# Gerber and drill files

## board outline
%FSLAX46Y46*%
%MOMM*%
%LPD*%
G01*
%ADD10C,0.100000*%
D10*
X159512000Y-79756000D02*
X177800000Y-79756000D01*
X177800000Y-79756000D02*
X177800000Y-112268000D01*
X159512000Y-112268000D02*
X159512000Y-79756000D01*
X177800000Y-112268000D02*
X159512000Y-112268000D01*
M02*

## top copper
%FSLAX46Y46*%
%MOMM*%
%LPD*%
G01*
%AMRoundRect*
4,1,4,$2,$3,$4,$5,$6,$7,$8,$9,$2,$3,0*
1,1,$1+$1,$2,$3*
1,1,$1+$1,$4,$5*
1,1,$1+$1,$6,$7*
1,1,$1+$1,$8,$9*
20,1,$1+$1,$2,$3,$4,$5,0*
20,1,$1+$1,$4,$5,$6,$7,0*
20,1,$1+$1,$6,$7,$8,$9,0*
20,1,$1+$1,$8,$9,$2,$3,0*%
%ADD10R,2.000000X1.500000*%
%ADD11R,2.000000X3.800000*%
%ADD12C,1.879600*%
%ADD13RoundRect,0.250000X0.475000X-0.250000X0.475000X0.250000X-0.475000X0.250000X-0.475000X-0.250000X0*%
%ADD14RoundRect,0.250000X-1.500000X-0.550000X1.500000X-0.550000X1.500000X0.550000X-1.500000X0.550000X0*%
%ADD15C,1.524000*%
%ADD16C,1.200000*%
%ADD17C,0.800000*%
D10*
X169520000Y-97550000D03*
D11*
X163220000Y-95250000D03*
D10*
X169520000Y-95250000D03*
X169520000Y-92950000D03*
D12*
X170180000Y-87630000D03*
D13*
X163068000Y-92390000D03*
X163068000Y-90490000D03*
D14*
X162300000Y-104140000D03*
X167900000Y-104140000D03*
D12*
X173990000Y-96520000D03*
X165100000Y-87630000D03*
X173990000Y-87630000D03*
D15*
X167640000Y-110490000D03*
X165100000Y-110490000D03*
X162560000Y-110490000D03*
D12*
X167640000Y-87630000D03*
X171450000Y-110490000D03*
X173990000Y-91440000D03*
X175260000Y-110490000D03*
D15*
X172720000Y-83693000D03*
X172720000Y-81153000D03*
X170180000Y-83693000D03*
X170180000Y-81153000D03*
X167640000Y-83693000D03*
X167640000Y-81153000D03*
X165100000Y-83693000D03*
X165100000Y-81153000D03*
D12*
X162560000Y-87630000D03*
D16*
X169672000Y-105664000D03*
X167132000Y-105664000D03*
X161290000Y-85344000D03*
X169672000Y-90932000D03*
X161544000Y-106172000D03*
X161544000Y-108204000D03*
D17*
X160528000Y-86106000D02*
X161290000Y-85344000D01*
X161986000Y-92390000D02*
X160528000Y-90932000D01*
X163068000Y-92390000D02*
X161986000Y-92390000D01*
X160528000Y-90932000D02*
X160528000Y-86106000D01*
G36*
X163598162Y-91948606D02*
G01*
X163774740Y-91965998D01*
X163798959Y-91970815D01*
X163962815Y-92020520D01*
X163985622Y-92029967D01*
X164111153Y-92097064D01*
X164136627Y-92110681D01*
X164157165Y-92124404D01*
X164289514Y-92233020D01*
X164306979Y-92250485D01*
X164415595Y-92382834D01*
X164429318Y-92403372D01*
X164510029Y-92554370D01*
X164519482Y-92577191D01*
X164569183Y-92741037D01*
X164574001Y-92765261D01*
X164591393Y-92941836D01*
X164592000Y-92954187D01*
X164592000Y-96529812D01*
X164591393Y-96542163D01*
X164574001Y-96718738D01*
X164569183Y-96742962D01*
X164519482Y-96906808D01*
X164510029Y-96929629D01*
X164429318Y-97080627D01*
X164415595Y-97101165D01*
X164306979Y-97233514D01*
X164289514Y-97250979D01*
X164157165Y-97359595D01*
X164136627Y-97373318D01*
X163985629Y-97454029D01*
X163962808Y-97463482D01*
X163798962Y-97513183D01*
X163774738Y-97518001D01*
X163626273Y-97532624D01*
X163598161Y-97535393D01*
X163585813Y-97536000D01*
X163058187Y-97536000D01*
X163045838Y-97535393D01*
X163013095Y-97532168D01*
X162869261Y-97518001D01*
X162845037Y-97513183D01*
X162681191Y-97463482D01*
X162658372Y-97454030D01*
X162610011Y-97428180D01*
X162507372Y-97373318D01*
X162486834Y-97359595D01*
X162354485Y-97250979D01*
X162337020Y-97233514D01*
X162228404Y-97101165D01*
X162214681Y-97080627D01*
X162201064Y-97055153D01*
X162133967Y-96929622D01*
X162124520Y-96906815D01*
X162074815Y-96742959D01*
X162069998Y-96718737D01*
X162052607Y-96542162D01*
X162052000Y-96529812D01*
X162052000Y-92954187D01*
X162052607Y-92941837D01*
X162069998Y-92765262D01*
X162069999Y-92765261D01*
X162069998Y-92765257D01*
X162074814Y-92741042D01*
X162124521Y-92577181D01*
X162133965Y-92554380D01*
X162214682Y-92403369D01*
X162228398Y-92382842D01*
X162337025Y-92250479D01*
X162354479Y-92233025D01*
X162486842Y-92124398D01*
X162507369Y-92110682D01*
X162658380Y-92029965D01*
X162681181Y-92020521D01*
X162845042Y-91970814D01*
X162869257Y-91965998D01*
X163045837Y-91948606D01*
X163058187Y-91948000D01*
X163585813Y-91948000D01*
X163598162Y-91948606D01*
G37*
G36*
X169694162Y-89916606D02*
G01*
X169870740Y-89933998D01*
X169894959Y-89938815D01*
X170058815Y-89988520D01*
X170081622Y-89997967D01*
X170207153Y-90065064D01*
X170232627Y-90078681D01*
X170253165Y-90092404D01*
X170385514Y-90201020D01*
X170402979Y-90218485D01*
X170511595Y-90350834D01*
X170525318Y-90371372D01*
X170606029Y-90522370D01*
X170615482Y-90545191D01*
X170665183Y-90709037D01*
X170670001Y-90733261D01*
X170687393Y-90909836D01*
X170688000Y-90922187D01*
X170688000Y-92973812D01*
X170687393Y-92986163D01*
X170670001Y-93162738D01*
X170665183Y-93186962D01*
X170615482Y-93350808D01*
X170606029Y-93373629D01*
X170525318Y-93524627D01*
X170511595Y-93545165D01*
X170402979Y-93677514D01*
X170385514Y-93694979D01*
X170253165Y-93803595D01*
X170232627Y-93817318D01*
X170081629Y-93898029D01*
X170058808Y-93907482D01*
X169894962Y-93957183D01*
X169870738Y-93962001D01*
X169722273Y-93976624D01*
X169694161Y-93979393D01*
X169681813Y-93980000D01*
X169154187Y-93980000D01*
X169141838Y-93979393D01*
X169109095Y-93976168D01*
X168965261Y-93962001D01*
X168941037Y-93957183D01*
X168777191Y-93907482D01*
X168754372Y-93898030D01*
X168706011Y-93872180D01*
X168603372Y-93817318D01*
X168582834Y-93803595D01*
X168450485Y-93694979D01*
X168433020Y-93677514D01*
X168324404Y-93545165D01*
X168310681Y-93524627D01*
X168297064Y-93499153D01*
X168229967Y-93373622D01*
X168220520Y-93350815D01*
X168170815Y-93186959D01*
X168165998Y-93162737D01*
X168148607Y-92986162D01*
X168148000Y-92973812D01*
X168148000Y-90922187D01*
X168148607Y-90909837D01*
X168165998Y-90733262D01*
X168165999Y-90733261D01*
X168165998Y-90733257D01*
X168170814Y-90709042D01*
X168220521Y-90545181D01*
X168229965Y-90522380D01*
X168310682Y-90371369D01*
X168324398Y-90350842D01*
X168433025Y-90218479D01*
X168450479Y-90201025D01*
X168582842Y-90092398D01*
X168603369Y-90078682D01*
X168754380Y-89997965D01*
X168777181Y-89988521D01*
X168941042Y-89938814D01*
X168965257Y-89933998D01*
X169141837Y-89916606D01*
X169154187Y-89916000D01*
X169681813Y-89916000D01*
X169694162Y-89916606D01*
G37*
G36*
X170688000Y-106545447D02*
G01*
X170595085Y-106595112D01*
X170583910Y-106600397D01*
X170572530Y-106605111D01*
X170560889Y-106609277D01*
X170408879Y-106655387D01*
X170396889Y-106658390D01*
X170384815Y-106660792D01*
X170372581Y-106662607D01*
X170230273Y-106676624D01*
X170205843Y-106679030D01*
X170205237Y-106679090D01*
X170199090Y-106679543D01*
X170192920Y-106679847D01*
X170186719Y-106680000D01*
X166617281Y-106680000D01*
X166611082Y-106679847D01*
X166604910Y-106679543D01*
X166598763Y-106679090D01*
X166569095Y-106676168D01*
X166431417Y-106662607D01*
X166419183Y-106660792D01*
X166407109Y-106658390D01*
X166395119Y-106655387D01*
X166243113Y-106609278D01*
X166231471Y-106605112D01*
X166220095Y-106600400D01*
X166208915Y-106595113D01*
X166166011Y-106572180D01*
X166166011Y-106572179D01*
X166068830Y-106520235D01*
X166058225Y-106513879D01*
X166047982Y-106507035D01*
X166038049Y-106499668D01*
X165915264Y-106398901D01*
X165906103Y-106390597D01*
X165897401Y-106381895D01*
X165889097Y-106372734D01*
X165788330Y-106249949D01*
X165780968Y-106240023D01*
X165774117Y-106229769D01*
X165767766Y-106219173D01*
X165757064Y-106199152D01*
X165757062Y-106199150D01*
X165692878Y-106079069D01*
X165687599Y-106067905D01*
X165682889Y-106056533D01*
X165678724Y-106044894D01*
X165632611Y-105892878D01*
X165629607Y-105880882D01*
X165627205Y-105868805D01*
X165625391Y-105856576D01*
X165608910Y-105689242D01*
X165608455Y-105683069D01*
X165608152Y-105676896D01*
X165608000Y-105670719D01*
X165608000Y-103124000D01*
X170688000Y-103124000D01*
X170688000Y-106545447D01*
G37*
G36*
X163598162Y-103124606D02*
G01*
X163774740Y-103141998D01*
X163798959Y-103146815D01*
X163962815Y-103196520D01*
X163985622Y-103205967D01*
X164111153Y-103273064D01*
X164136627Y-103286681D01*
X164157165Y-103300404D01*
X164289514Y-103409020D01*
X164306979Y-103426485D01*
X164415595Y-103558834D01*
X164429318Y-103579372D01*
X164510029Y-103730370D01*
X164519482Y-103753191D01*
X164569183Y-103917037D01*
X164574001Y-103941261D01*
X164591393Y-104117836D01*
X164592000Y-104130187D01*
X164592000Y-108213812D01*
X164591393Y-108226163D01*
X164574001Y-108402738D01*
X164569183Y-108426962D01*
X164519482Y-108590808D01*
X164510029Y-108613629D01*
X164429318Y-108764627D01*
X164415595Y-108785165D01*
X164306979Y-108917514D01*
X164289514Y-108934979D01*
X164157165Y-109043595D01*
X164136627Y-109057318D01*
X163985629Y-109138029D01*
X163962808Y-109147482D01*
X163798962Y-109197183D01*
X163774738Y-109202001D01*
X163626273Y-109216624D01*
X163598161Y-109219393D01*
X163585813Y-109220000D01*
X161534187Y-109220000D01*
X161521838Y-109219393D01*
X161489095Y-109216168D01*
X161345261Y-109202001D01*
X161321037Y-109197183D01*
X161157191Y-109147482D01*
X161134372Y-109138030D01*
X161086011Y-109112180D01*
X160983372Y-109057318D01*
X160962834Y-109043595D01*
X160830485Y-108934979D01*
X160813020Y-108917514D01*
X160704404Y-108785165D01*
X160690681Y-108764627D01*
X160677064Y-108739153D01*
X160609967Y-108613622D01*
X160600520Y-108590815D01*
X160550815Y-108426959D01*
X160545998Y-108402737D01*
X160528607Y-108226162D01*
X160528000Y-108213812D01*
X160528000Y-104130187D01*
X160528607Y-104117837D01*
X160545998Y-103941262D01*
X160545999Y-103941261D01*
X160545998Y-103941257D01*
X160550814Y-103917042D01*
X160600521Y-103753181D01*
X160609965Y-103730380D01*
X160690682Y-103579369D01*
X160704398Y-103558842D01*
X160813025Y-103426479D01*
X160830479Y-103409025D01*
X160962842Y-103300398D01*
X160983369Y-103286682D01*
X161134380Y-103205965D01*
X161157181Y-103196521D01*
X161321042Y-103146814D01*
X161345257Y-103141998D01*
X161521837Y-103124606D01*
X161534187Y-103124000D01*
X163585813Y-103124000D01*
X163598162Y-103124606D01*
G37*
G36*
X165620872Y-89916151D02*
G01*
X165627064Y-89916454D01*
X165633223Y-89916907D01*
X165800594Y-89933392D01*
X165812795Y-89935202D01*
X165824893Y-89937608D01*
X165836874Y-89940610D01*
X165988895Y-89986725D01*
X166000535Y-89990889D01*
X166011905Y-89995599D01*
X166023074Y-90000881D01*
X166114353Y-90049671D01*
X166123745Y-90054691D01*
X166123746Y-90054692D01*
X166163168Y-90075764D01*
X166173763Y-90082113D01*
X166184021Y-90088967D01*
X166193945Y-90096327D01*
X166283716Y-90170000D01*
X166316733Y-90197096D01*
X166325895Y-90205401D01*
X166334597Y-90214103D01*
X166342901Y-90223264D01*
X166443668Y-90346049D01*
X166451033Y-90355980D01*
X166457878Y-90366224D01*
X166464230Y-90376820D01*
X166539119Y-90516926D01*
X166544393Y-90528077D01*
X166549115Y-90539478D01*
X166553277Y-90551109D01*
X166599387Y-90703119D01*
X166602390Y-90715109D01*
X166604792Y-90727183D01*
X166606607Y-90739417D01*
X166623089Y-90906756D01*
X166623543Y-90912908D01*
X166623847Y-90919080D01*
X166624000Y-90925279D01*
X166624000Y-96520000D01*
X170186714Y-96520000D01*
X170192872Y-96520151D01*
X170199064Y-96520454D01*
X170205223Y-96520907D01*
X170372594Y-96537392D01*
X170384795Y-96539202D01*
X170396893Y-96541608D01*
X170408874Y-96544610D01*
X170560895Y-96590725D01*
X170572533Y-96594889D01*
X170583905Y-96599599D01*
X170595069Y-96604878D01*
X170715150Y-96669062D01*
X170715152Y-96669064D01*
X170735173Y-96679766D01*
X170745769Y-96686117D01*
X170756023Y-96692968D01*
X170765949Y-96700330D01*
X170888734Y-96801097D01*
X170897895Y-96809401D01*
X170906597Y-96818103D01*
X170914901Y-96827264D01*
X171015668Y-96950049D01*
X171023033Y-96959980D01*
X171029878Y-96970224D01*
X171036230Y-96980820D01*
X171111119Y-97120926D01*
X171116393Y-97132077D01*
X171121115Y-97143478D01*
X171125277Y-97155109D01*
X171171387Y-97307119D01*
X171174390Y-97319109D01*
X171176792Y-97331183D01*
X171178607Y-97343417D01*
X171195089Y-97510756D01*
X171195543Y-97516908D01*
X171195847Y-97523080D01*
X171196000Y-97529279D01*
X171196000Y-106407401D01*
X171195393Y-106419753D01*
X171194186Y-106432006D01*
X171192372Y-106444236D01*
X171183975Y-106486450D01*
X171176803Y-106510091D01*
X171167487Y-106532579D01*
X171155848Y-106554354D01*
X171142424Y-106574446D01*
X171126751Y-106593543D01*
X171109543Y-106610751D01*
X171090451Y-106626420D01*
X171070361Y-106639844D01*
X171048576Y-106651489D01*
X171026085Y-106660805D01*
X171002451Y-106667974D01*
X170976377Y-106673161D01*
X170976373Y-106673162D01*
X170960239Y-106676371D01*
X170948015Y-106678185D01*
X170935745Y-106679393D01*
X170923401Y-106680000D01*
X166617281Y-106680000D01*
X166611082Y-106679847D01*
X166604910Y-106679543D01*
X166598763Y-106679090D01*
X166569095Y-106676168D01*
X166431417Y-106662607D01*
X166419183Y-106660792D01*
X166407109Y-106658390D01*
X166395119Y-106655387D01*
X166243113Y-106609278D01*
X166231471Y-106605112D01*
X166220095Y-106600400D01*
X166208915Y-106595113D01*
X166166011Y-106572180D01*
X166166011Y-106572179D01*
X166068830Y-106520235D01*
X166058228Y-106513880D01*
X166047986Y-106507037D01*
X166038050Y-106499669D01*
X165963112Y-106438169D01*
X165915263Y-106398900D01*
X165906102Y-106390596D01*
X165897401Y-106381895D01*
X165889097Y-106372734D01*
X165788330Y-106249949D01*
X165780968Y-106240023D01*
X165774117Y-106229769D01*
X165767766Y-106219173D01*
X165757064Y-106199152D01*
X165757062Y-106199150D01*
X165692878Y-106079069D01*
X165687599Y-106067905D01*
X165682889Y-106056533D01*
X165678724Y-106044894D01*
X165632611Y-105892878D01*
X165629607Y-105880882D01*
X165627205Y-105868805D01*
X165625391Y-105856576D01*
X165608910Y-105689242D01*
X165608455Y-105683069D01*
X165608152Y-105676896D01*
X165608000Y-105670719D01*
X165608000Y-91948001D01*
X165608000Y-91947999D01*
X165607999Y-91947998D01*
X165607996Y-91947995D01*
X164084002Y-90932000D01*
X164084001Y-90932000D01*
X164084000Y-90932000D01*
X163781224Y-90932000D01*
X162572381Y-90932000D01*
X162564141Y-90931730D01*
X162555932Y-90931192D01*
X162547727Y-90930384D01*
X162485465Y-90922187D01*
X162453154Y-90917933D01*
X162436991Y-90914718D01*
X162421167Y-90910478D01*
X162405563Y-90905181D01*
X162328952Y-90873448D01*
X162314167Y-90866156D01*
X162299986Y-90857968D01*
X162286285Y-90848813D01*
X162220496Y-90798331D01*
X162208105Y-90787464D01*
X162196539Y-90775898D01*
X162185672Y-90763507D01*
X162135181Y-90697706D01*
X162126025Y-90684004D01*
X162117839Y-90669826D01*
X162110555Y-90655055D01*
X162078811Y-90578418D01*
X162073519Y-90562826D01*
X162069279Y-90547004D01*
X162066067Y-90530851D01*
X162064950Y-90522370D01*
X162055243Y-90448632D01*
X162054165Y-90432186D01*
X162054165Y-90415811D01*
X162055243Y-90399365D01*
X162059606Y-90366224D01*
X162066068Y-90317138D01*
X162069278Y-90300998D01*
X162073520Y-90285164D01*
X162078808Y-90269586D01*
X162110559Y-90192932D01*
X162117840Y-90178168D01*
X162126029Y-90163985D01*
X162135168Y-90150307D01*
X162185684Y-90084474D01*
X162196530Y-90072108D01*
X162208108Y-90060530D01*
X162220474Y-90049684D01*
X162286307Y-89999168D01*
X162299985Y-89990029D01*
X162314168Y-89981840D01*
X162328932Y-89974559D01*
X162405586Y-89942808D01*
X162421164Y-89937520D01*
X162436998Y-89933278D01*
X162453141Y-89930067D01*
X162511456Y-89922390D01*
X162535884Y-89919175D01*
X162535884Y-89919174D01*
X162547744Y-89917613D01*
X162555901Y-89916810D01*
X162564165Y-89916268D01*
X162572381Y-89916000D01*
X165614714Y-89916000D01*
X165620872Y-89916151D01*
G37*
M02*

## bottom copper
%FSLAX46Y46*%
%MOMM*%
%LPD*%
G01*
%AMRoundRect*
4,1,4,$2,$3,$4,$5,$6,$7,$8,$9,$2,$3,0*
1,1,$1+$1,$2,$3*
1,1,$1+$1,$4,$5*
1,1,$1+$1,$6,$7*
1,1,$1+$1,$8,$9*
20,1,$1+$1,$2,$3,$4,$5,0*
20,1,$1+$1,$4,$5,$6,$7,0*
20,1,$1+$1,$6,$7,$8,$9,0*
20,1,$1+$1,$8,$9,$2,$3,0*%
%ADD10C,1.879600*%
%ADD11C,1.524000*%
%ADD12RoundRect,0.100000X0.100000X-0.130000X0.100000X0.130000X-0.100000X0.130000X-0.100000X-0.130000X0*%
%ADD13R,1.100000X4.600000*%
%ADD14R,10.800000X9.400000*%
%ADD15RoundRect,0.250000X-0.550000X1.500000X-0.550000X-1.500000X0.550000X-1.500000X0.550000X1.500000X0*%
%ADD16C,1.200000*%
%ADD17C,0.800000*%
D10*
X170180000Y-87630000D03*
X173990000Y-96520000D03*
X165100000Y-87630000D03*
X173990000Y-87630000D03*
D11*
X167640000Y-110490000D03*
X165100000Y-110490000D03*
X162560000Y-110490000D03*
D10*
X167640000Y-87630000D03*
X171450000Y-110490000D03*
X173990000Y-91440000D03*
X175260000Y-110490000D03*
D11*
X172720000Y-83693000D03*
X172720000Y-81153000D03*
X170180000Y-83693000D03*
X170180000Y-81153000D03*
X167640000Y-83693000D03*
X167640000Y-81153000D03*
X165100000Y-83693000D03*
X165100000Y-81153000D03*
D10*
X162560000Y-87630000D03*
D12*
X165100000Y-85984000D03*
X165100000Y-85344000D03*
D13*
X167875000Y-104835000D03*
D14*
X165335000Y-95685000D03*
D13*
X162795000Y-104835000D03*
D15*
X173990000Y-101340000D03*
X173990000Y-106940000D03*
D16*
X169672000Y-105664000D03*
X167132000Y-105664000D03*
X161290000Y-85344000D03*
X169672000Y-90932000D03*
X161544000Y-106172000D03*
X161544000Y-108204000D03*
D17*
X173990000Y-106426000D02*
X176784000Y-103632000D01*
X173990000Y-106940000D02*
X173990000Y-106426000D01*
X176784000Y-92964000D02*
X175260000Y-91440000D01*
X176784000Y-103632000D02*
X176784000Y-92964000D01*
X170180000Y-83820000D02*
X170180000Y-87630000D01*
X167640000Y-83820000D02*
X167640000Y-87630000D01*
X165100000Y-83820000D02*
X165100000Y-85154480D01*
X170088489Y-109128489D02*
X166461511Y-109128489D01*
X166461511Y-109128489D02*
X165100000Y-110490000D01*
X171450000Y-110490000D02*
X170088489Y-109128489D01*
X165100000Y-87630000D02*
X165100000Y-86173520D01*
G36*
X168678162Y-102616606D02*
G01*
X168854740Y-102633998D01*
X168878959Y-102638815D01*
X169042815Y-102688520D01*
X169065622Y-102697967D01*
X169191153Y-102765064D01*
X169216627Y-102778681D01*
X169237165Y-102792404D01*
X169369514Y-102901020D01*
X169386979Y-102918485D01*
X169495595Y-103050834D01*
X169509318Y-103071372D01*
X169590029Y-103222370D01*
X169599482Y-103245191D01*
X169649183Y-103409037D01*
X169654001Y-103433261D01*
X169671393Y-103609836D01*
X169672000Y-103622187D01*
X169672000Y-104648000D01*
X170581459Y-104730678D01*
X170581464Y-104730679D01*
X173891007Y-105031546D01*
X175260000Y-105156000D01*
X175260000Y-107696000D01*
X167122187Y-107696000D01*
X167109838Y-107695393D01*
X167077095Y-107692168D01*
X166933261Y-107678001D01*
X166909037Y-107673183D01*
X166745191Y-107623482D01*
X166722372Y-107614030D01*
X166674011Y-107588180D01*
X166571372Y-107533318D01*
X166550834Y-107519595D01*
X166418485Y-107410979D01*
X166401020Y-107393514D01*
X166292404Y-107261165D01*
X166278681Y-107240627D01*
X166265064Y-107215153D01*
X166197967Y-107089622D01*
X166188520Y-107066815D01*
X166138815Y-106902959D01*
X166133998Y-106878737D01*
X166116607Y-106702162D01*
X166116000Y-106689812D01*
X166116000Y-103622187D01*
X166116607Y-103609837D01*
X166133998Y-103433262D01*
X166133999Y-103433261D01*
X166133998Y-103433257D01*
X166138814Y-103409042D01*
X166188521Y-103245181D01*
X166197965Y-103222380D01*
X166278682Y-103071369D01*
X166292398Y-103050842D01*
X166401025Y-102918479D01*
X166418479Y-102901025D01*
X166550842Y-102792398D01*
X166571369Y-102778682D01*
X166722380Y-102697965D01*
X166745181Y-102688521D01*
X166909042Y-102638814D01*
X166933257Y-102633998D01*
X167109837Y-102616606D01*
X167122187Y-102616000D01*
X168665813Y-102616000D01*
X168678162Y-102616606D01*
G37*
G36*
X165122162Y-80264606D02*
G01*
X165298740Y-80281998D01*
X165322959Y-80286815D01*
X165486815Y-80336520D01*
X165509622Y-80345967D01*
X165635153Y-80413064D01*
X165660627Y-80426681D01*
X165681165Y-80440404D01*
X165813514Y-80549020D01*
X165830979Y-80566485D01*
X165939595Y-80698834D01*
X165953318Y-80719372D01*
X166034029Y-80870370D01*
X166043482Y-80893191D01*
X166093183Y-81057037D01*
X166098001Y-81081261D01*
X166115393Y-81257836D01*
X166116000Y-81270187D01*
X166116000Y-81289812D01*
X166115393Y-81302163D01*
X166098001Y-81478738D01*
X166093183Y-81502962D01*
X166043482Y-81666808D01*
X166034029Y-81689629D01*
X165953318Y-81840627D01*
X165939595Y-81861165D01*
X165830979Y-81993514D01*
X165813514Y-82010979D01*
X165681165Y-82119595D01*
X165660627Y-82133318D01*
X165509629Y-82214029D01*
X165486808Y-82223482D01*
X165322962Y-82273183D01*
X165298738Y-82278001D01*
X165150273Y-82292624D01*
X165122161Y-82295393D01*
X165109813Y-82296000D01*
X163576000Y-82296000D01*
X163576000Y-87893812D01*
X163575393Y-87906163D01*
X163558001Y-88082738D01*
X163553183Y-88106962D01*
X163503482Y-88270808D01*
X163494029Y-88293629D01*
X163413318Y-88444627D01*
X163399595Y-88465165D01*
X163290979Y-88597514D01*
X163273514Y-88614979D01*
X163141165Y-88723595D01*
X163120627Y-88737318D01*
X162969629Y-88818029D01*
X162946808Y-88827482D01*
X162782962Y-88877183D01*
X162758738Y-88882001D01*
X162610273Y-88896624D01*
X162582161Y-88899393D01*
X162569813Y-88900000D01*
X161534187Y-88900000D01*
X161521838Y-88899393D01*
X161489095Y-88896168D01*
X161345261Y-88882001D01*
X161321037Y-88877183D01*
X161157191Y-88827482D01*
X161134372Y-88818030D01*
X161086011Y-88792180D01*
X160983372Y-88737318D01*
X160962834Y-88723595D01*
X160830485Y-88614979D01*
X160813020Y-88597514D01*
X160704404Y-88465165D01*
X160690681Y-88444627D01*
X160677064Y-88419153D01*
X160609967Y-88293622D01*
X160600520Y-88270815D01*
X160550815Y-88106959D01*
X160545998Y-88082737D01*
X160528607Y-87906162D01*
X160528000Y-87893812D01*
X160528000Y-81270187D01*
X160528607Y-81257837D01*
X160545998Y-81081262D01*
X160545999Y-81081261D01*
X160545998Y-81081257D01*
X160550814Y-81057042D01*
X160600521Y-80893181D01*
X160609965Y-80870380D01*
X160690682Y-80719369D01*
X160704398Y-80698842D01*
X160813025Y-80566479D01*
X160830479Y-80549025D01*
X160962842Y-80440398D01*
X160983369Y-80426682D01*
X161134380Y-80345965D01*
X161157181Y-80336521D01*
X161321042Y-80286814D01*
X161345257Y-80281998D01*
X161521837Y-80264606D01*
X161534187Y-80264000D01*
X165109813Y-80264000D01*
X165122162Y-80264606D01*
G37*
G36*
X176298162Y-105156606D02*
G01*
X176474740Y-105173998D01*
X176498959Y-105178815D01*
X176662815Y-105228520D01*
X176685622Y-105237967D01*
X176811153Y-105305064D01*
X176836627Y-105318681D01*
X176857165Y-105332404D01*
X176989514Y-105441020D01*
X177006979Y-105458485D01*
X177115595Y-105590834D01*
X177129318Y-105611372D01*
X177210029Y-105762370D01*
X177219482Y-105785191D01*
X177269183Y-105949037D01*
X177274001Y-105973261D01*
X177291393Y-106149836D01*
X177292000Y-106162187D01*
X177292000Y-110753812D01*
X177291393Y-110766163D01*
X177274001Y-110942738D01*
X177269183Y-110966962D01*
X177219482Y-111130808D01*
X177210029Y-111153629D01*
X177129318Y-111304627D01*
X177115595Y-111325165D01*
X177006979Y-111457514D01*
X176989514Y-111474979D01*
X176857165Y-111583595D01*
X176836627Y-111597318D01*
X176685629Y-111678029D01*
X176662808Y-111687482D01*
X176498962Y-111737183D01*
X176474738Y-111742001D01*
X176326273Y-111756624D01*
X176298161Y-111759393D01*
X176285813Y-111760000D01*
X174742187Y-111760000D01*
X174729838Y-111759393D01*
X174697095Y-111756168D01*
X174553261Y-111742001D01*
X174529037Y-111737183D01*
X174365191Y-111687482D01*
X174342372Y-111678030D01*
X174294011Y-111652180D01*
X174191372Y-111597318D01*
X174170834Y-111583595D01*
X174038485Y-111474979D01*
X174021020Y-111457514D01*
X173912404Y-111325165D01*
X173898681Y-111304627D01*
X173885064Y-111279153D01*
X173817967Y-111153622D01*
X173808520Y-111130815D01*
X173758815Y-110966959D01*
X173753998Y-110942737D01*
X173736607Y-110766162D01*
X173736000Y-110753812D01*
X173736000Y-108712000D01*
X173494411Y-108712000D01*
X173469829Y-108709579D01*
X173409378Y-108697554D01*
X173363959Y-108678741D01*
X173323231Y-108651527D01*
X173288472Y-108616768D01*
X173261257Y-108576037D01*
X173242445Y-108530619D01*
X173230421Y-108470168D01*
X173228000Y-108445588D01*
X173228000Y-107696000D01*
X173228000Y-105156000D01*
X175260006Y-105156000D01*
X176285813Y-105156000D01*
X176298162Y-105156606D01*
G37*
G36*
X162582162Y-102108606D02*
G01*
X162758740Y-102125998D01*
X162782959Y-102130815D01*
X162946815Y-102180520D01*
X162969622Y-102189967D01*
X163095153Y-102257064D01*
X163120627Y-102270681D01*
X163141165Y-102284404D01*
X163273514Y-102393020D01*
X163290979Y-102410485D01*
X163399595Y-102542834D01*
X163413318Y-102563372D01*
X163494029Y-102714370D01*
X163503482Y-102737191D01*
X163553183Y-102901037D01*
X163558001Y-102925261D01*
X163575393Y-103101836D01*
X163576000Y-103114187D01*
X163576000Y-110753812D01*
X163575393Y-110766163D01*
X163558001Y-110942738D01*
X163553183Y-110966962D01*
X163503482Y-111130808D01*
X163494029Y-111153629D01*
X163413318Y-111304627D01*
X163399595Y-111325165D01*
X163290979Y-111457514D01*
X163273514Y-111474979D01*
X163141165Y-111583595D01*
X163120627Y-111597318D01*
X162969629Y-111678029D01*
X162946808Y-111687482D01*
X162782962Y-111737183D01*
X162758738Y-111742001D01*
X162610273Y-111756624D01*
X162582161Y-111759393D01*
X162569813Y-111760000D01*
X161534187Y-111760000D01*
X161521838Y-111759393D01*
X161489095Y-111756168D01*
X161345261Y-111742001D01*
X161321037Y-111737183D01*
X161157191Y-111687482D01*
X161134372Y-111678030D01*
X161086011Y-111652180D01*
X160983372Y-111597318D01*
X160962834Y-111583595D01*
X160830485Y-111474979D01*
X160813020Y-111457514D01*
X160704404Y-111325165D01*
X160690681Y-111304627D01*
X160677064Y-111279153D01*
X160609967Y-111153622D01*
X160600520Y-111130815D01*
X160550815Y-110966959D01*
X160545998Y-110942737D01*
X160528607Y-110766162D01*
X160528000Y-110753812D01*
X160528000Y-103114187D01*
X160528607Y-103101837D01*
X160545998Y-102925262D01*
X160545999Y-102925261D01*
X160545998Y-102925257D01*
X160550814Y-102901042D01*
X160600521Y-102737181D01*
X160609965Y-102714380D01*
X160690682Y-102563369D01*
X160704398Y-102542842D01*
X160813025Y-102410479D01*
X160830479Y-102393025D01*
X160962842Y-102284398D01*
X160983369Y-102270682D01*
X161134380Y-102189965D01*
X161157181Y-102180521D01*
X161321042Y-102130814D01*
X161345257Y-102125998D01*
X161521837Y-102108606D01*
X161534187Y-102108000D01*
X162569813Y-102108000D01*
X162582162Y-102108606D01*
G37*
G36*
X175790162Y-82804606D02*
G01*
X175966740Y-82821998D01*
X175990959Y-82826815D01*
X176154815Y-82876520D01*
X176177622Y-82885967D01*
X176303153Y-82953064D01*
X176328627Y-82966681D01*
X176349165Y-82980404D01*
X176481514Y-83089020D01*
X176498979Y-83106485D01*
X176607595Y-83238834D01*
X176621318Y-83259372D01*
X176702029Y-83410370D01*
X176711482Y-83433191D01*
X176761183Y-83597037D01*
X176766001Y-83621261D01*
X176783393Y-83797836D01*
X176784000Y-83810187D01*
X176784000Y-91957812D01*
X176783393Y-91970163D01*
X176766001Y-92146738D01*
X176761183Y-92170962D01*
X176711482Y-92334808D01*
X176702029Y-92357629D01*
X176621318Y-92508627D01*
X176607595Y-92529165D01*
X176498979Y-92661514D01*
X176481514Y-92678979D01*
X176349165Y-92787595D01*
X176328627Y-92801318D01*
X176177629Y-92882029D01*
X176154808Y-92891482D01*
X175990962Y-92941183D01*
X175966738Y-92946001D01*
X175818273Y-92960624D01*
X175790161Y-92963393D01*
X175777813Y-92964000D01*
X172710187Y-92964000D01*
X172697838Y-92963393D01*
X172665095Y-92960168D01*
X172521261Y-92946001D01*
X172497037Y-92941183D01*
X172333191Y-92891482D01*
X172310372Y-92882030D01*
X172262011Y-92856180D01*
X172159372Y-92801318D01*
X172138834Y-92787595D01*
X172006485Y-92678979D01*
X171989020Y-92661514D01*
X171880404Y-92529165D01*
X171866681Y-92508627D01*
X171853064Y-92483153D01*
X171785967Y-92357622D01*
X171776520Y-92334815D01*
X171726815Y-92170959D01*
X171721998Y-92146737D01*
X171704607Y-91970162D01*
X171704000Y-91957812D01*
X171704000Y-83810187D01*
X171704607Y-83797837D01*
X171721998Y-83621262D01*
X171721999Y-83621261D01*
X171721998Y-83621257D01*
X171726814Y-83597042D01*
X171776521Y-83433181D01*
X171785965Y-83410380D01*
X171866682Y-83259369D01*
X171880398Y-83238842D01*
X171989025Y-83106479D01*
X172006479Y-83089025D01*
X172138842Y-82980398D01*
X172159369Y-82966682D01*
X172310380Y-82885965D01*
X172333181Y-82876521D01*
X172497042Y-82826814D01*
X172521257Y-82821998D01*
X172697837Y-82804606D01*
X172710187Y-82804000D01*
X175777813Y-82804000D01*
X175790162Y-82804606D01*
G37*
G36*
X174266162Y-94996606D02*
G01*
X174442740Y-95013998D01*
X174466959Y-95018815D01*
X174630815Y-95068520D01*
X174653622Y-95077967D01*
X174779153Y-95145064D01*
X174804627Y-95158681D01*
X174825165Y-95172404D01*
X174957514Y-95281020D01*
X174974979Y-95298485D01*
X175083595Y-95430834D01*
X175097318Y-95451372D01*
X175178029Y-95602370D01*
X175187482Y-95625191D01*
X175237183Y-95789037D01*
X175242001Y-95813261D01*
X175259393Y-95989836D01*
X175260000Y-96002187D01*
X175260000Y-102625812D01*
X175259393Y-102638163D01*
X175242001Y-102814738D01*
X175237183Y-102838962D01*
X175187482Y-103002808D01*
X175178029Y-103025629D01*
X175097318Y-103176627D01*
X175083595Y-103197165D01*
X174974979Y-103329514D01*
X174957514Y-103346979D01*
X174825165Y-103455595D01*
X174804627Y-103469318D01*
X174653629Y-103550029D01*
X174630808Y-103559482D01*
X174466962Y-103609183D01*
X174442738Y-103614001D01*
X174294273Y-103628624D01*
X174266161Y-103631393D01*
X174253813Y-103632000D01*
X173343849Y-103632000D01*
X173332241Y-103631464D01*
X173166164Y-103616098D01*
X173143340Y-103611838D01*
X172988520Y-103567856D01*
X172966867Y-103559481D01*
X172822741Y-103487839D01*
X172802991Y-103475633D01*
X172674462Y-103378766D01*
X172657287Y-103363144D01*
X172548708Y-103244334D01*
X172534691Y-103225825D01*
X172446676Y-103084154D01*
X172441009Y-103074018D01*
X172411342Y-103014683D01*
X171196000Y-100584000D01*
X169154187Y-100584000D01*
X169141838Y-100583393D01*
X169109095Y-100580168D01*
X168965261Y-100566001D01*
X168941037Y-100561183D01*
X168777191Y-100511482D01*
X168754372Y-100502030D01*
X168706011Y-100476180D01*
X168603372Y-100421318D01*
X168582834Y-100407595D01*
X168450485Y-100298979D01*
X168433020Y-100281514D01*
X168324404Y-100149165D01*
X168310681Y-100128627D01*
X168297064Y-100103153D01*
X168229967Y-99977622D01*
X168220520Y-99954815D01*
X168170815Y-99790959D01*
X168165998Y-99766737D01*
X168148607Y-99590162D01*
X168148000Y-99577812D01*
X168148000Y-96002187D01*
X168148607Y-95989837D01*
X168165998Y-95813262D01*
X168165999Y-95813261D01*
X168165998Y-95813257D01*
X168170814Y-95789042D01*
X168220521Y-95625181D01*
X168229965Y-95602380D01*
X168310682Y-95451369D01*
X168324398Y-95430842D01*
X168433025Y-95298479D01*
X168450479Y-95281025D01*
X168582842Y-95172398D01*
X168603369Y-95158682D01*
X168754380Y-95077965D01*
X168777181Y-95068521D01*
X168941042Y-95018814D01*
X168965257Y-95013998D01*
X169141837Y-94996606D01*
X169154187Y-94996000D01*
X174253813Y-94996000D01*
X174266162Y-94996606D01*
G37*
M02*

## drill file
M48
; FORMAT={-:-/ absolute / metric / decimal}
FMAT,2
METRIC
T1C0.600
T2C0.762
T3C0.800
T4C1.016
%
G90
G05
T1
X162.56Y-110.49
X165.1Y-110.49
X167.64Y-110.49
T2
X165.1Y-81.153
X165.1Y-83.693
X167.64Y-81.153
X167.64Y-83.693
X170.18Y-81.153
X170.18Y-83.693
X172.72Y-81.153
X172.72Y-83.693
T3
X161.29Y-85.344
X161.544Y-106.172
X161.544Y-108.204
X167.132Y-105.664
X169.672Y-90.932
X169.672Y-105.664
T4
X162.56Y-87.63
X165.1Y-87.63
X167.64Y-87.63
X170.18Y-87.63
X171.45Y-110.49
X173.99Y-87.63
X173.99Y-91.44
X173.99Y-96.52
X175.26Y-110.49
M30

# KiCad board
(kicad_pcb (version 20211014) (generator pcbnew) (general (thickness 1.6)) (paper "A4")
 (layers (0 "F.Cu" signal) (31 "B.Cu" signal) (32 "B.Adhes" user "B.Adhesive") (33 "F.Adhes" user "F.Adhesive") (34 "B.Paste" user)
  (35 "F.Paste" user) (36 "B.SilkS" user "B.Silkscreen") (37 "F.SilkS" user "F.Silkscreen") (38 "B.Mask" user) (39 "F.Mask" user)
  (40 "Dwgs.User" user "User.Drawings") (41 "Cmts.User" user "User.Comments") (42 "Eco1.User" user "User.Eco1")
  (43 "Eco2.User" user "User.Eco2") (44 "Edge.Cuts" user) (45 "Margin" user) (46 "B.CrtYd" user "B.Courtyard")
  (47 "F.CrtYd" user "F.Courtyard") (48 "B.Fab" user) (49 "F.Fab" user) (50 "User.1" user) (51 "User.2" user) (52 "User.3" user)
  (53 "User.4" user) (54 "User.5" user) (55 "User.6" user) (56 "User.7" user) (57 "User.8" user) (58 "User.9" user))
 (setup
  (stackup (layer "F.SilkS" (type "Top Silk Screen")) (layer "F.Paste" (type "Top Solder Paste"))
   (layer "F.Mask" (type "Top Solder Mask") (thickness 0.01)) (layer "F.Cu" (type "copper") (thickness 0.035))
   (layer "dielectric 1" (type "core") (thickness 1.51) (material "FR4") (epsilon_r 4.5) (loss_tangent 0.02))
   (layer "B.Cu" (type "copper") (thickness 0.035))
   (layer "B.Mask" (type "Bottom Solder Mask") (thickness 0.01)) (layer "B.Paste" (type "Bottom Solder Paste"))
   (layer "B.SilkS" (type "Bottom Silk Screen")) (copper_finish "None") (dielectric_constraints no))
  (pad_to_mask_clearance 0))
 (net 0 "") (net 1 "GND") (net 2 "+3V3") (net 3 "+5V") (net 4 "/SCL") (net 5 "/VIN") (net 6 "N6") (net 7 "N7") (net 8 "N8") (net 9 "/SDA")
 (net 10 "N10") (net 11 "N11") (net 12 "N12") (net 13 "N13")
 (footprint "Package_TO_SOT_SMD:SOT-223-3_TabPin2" (layer "F.Cu") (at 166.37 95.25 180)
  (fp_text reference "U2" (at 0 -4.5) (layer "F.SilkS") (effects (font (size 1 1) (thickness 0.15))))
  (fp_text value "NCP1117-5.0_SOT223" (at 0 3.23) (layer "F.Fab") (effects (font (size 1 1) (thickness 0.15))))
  (pad "1" smd rect (at -3.15 -2.3 180) (size 2 1.5) (layers "F.Cu" "F.Paste" "F.Mask") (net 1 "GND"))
  (pad "2" smd rect (at 3.15 0 180) (size 2 3.8) (layers "F.Cu" "F.Paste" "F.Mask") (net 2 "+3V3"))
  (pad "2" smd rect (at -3.15 0 180) (size 2 1.5) (layers "F.Cu" "F.Paste" "F.Mask") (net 2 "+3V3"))
  (pad "3" smd rect (at -3.15 2.3 180) (size 2 1.5) (layers "F.Cu" "F.Paste" "F.Mask") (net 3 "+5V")))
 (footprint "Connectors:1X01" (layer "F.Cu") (at 170.18 87.63 180)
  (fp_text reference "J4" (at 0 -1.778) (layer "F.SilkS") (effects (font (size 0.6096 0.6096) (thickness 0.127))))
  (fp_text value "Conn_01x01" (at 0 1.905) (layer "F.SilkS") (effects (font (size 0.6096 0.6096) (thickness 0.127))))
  (pad "1" thru_hole circle locked (at 0 0 180) (size 1.8796 1.8796) (drill 1.016) (layers *.Cu *.Mask) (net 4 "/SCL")
   (solder_mask_margin 0.1016)))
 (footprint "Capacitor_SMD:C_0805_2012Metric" (layer "F.Cu") (at 163.068 91.44 90)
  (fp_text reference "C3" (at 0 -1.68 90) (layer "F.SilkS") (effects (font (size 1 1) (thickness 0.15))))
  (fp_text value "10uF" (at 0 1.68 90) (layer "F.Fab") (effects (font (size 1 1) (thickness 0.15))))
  (pad "1" smd roundrect (at -0.95 0 90) (size 1 1.45) (layers "F.Cu" "F.Paste" "F.Mask") (roundrect_rratio 0.25) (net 2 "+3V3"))
  (pad "2" smd roundrect (at 0.95 0 90) (size 1 1.45) (layers "F.Cu" "F.Paste" "F.Mask") (roundrect_rratio 0.25) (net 1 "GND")))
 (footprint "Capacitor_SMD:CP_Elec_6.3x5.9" (layer "F.Cu") (at 165.1 104.14)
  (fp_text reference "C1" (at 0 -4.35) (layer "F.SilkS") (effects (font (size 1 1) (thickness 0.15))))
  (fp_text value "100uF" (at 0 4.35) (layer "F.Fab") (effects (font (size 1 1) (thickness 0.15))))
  (pad "1" smd roundrect (at -2.8 0) (size 3.5 1.6) (layers "F.Cu" "F.Paste" "F.Mask") (roundrect_rratio 0.15625) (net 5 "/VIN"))
  (pad "2" smd roundrect (at 2.8 0) (size 3.5 1.6) (layers "F.Cu" "F.Paste" "F.Mask") (roundrect_rratio 0.15625) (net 1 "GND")))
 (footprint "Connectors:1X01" (layer "F.Cu") (at 173.99 96.52)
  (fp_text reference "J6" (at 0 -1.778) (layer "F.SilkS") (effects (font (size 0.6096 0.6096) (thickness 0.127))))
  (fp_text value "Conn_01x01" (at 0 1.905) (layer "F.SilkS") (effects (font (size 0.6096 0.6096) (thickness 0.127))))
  (pad "1" thru_hole circle locked (at 0 0) (size 1.8796 1.8796) (drill 1.016) (layers *.Cu *.Mask) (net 3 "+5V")
   (solder_mask_margin 0.1016)))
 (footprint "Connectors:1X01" (layer "F.Cu") (at 165.1 87.63 180)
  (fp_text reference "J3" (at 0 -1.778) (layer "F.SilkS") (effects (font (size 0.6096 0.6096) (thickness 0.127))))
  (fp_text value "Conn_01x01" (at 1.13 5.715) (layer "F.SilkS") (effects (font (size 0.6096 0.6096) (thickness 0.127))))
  (pad "1" thru_hole circle locked (at 0 0 180) (size 1.8796 1.8796) (drill 1.016) (layers *.Cu *.Mask) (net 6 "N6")
   (solder_mask_margin 0.1016)))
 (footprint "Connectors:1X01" (layer "F.Cu") (at 173.99 87.63)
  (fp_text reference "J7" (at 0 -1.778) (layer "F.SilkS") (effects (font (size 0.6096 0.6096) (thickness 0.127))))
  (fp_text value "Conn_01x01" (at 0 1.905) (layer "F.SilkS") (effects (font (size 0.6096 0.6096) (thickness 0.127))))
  (pad "1" thru_hole circle locked (at 0 0) (size 1.8796 1.8796) (drill 1.016) (layers *.Cu *.Mask) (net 1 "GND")
   (solder_mask_margin 0.1016)))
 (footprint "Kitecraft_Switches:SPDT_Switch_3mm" (layer "F.Cu") (at 165.1 110.49 180)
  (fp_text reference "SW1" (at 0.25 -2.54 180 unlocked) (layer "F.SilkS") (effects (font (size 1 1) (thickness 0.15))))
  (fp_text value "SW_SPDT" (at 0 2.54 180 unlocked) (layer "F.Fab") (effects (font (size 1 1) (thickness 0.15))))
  (pad "1" thru_hole circle (at -2.54 0 180) (size 1.524 1.524) (drill 0.6) (layers *.Cu *.Mask) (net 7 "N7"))
  (pad "2" thru_hole circle (at 0 0 180) (size 1.524 1.524) (drill 0.6) (layers *.Cu *.Mask) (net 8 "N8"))
  (pad "3" thru_hole circle (at 2.54 0 180) (size 1.524 1.524) (drill 0.6) (layers *.Cu *.Mask) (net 5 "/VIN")))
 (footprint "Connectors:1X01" (layer "F.Cu") (at 167.64 87.63 180)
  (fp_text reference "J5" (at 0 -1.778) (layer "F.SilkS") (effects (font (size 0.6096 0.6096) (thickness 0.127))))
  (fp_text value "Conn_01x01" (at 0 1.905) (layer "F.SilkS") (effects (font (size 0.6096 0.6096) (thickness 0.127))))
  (pad "1" thru_hole circle locked (at 0 0 180) (size 1.8796 1.8796) (drill 1.016) (layers *.Cu *.Mask) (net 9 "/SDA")
   (solder_mask_margin 0.1016)))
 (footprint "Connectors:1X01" (layer "F.Cu") (at 171.45 110.49 180)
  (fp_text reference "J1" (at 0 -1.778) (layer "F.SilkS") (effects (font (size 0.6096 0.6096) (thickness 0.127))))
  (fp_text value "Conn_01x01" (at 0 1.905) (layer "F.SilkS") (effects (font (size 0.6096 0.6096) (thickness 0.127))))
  (pad "1" thru_hole circle locked (at 0 0 180) (size 1.8796 1.8796) (drill 1.016) (layers *.Cu *.Mask) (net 8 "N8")
   (solder_mask_margin 0.1016)))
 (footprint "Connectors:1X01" (layer "F.Cu") (at 173.99 91.44)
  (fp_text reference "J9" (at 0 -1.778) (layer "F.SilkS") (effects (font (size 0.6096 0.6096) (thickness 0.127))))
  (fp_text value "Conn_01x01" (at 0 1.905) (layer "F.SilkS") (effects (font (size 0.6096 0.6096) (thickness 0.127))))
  (pad "1" thru_hole circle locked (at 0 0) (size 1.8796 1.8796) (drill 1.016) (layers *.Cu *.Mask) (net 1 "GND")
   (solder_mask_margin 0.1016)))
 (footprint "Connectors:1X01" (layer "F.Cu") (at 175.26 110.49 180)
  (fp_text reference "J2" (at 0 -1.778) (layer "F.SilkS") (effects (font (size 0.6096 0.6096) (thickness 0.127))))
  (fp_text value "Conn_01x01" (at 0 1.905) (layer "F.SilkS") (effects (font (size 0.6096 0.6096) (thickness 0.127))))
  (pad "1" thru_hole circle locked (at 0 0 180) (size 1.8796 1.8796) (drill 1.016) (layers *.Cu *.Mask) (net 1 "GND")
   (solder_mask_margin 0.1016)))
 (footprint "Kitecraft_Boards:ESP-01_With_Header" (layer "F.Cu") (at 168.91 82.423 180)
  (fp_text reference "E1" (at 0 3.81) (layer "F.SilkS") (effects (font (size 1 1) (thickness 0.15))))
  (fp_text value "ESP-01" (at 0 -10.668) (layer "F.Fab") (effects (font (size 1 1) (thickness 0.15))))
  (pad "1" thru_hole circle locked (at -3.81 -1.27 180) (size 1.524 1.524) (drill 0.762) (layers *.Cu *.Mask) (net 1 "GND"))
  (pad "2" thru_hole circle locked (at -3.81 1.27 180) (size 1.524 1.524) (drill 0.762) (layers *.Cu *.Mask) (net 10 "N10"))
  (pad "3" thru_hole circle locked (at -1.27 -1.27 180) (size 1.524 1.524) (drill 0.762) (layers *.Cu *.Mask) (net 4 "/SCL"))
  (pad "4" thru_hole circle locked (at -1.27 1.27 180) (size 1.524 1.524) (drill 0.762) (layers *.Cu *.Mask) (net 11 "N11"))
  (pad "5" thru_hole circle locked (at 1.27 -1.27 180) (size 1.524 1.524) (drill 0.762) (layers *.Cu *.Mask) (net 9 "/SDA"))
  (pad "6" thru_hole circle locked (at 1.27 1.27 180) (size 1.524 1.524) (drill 0.762) (layers *.Cu *.Mask) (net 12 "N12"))
  (pad "7" thru_hole circle locked (at 3.81 -1.27 180) (size 1.524 1.524) (drill 0.762) (layers *.Cu *.Mask) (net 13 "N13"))
  (pad "8" thru_hole circle locked (at 3.81 1.27 180) (size 1.524 1.524) (drill 0.762) (layers *.Cu *.Mask) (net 2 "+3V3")))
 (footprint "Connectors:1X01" (layer "F.Cu") (at 162.56 87.63)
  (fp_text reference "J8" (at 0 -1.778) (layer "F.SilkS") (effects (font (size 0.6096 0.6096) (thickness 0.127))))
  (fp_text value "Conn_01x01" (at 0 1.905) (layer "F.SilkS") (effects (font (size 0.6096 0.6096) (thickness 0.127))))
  (pad "1" thru_hole circle locked (at 0 0) (size 1.8796 1.8796) (drill 1.016) (layers *.Cu *.Mask) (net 2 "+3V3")
   (solder_mask_margin 0.1016)))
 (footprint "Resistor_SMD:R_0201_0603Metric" (layer "B.Cu") (at 165.1 85.664 90)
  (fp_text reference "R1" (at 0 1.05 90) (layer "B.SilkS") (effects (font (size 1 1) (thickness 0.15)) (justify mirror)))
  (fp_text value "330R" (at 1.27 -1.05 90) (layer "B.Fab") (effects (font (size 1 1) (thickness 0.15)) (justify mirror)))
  (pad "" smd roundrect (at 0.345 0 90) (size 0.318 0.36) (layers "B.Paste") (roundrect_rratio 0.25))
  (pad "" smd roundrect (at -0.345 0 90) (size 0.318 0.36) (layers "B.Paste") (roundrect_rratio 0.25))
  (pad "1" smd roundrect (at -0.32 0 90) (size 0.46 0.4) (layers "B.Cu" "B.Mask") (roundrect_rratio 0.25) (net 6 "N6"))
  (pad "2" smd roundrect (at 0.32 0 90) (size 0.46 0.4) (layers "B.Cu" "B.Mask") (roundrect_rratio 0.25) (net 13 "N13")))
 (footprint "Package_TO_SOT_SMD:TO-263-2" (layer "B.Cu") (at 165.335 99.06 90)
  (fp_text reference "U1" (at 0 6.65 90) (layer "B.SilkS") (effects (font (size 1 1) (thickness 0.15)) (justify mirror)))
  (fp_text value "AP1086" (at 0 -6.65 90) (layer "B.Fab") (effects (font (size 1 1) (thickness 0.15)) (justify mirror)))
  (pad "" smd rect (at 5.8 -2.775 90) (size 4.55 5.25) (layers "B.Paste"))
  (pad "" smd rect (at 0.95 2.775 90) (size 4.55 5.25) (layers "B.Paste"))
  (pad "" smd rect (at 5.8 2.775 90) (size 4.55 5.25) (layers "B.Paste"))
  (pad "" smd rect (at 0.95 -2.775 90) (size 4.55 5.25) (layers "B.Paste"))
  (pad "1" smd rect (at -5.775 2.54 90) (size 4.6 1.1) (layers "B.Cu" "B.Paste" "B.Mask") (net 1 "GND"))
  (pad "2" smd rect (at 3.375 0 90) (size 9.4 10.8) (layers "B.Cu" "B.Mask") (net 3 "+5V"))
  (pad "3" smd rect (at -5.775 -2.54 90) (size 4.6 1.1) (layers "B.Cu" "B.Paste" "B.Mask") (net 5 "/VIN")))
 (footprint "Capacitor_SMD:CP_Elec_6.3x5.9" (layer "B.Cu") (at 173.99 104.14 -90)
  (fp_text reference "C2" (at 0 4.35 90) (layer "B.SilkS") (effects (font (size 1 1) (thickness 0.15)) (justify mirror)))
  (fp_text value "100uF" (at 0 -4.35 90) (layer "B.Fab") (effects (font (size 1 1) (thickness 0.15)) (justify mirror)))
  (pad "1" smd roundrect (at -2.8 0 270) (size 3.5 1.6) (layers "B.Cu" "B.Paste" "B.Mask") (roundrect_rratio 0.15625) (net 3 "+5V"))
  (pad "2" smd roundrect (at 2.8 0 270) (size 3.5 1.6) (layers "B.Cu" "B.Paste" "B.Mask") (roundrect_rratio 0.15625) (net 1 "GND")))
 (gr_line (start 159.512 79.756) (end 177.8 79.756) (layer "Edge.Cuts") (width 0.1))
 (gr_line (start 177.8 79.756) (end 177.8 112.268) (layer "Edge.Cuts") (width 0.1))
 (gr_line (start 159.512 112.268) (end 159.512 79.756) (layer "Edge.Cuts") (width 0.1))
 (gr_line (start 177.8 112.268) (end 159.512 112.268) (layer "Edge.Cuts") (width 0.1))
 (via (at 169.672 105.664) (size 1.2) (drill 0.8) (layers "F.Cu" "B.Cu") (free) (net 1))
 (via (at 167.132 105.664) (size 1.2) (drill 0.8) (layers "F.Cu" "B.Cu") (free) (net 1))
 (segment (start 173.99 106.426) (end 176.784 103.632) (width 0.8) (layer "B.Cu") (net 1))
 (segment (start 173.99 106.94) (end 173.99 106.426) (width 0.8) (layer "B.Cu") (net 1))
 (segment (start 176.784 92.964) (end 175.26 91.44) (width 0.8) (layer "B.Cu") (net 1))
 (segment (start 176.784 103.632) (end 176.784 92.964) (width 0.8) (layer "B.Cu") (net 1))
 (segment (start 170.18 83.82) (end 170.18 87.63) (width 0.8) (layer "B.Cu") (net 4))
 (segment (start 167.64 83.82) (end 167.64 87.63) (width 0.8) (layer "B.Cu") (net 9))
 (segment (start 165.1 83.82) (end 165.1 85.15448) (width 0.8) (layer "B.Cu") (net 13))
 (segment (start 160.528 86.106) (end 161.29 85.344) (width 0.8) (layer "F.Cu") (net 2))
 (segment (start 161.986 92.39) (end 160.528 90.932) (width 0.8) (layer "F.Cu") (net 2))
 (segment (start 163.068 92.39) (end 161.986 92.39) (width 0.8) (layer "F.Cu") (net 2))
 (segment (start 160.528 90.932) (end 160.528 86.106) (width 0.8) (layer "F.Cu") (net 2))
 (via (at 161.29 85.344) (size 1.2) (drill 0.8) (layers "F.Cu" "B.Cu") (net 2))
 (via (at 169.672 90.932) (size 1.2) (drill 0.8) (layers "F.Cu" "B.Cu") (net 3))
 (via (at 161.544 106.172) (size 1.2) (drill 0.8) (layers "F.Cu" "B.Cu") (free) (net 5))
 (via (at 161.544 108.204) (size 1.2) (drill 0.8) (layers "F.Cu" "B.Cu") (free) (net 5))
 (segment (start 170.088489 109.128489) (end 166.461511 109.128489) (width 0.8) (layer "B.Cu") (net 8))
 (segment (start 166.461511 109.128489) (end 165.1 110.49) (width 0.8) (layer "B.Cu") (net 8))
 (segment (start 171.45 110.49) (end 170.088489 109.128489) (width 0.8) (layer "B.Cu") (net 8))
 (segment (start 165.1 87.63) (end 165.1 86.17352) (width 0.8) (layer "B.Cu") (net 6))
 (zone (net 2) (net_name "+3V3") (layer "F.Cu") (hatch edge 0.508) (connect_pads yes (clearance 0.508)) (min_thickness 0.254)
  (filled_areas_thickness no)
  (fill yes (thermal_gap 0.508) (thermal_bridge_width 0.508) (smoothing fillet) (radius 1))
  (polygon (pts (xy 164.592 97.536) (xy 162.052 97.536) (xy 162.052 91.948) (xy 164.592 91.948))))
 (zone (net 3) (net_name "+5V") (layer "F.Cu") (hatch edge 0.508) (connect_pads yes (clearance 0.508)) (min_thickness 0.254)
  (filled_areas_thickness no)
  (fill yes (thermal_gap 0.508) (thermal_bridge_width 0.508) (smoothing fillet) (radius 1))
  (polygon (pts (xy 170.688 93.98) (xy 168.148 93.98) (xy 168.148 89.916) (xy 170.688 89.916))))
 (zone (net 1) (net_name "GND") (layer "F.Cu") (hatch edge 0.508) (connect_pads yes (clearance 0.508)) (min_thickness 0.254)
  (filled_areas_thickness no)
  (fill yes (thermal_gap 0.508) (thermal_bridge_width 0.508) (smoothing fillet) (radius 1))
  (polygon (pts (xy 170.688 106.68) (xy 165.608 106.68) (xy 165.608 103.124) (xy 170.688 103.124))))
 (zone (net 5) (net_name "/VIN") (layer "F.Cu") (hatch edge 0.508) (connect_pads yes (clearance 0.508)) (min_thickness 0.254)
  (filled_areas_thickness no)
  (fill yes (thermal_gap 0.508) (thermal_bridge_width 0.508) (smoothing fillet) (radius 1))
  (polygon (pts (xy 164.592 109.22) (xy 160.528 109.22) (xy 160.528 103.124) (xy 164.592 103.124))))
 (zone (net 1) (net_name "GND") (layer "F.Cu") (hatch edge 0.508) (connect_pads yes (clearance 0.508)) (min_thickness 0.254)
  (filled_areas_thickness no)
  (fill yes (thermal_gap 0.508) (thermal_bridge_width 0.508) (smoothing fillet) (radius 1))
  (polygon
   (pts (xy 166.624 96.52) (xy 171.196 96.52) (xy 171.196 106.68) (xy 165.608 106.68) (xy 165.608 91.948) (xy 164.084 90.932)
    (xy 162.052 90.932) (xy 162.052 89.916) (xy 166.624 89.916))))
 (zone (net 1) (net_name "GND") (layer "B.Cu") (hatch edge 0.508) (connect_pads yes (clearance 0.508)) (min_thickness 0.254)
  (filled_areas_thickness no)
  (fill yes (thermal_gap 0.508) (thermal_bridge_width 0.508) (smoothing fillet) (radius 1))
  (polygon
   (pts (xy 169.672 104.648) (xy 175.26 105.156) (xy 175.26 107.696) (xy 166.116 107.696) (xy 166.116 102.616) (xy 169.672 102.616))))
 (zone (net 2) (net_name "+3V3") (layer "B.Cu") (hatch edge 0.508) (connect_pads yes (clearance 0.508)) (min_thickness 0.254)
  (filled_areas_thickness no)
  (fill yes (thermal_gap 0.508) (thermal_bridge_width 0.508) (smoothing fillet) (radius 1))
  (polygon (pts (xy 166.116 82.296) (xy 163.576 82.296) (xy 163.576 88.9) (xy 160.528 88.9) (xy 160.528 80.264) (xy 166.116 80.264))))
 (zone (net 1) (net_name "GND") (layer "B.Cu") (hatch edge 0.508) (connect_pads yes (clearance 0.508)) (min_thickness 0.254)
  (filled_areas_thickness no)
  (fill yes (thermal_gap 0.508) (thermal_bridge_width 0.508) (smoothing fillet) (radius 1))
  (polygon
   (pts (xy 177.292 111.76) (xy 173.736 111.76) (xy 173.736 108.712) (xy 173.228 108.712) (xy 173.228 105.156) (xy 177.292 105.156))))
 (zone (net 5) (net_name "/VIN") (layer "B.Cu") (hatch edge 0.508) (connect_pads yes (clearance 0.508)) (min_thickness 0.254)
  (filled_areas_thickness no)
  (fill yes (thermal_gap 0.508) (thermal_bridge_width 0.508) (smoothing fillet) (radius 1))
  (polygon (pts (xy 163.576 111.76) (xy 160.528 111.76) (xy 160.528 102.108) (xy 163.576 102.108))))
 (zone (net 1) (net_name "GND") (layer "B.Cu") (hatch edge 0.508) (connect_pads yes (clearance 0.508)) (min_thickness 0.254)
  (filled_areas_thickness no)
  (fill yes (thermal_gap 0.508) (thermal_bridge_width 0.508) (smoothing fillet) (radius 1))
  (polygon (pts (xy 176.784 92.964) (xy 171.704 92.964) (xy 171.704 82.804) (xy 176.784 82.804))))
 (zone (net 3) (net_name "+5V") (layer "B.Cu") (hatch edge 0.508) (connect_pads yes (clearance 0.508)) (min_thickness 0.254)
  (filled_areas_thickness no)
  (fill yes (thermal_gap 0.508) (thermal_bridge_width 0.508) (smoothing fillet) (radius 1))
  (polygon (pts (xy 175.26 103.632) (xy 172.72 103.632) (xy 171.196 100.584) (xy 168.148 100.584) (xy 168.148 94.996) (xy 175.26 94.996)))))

